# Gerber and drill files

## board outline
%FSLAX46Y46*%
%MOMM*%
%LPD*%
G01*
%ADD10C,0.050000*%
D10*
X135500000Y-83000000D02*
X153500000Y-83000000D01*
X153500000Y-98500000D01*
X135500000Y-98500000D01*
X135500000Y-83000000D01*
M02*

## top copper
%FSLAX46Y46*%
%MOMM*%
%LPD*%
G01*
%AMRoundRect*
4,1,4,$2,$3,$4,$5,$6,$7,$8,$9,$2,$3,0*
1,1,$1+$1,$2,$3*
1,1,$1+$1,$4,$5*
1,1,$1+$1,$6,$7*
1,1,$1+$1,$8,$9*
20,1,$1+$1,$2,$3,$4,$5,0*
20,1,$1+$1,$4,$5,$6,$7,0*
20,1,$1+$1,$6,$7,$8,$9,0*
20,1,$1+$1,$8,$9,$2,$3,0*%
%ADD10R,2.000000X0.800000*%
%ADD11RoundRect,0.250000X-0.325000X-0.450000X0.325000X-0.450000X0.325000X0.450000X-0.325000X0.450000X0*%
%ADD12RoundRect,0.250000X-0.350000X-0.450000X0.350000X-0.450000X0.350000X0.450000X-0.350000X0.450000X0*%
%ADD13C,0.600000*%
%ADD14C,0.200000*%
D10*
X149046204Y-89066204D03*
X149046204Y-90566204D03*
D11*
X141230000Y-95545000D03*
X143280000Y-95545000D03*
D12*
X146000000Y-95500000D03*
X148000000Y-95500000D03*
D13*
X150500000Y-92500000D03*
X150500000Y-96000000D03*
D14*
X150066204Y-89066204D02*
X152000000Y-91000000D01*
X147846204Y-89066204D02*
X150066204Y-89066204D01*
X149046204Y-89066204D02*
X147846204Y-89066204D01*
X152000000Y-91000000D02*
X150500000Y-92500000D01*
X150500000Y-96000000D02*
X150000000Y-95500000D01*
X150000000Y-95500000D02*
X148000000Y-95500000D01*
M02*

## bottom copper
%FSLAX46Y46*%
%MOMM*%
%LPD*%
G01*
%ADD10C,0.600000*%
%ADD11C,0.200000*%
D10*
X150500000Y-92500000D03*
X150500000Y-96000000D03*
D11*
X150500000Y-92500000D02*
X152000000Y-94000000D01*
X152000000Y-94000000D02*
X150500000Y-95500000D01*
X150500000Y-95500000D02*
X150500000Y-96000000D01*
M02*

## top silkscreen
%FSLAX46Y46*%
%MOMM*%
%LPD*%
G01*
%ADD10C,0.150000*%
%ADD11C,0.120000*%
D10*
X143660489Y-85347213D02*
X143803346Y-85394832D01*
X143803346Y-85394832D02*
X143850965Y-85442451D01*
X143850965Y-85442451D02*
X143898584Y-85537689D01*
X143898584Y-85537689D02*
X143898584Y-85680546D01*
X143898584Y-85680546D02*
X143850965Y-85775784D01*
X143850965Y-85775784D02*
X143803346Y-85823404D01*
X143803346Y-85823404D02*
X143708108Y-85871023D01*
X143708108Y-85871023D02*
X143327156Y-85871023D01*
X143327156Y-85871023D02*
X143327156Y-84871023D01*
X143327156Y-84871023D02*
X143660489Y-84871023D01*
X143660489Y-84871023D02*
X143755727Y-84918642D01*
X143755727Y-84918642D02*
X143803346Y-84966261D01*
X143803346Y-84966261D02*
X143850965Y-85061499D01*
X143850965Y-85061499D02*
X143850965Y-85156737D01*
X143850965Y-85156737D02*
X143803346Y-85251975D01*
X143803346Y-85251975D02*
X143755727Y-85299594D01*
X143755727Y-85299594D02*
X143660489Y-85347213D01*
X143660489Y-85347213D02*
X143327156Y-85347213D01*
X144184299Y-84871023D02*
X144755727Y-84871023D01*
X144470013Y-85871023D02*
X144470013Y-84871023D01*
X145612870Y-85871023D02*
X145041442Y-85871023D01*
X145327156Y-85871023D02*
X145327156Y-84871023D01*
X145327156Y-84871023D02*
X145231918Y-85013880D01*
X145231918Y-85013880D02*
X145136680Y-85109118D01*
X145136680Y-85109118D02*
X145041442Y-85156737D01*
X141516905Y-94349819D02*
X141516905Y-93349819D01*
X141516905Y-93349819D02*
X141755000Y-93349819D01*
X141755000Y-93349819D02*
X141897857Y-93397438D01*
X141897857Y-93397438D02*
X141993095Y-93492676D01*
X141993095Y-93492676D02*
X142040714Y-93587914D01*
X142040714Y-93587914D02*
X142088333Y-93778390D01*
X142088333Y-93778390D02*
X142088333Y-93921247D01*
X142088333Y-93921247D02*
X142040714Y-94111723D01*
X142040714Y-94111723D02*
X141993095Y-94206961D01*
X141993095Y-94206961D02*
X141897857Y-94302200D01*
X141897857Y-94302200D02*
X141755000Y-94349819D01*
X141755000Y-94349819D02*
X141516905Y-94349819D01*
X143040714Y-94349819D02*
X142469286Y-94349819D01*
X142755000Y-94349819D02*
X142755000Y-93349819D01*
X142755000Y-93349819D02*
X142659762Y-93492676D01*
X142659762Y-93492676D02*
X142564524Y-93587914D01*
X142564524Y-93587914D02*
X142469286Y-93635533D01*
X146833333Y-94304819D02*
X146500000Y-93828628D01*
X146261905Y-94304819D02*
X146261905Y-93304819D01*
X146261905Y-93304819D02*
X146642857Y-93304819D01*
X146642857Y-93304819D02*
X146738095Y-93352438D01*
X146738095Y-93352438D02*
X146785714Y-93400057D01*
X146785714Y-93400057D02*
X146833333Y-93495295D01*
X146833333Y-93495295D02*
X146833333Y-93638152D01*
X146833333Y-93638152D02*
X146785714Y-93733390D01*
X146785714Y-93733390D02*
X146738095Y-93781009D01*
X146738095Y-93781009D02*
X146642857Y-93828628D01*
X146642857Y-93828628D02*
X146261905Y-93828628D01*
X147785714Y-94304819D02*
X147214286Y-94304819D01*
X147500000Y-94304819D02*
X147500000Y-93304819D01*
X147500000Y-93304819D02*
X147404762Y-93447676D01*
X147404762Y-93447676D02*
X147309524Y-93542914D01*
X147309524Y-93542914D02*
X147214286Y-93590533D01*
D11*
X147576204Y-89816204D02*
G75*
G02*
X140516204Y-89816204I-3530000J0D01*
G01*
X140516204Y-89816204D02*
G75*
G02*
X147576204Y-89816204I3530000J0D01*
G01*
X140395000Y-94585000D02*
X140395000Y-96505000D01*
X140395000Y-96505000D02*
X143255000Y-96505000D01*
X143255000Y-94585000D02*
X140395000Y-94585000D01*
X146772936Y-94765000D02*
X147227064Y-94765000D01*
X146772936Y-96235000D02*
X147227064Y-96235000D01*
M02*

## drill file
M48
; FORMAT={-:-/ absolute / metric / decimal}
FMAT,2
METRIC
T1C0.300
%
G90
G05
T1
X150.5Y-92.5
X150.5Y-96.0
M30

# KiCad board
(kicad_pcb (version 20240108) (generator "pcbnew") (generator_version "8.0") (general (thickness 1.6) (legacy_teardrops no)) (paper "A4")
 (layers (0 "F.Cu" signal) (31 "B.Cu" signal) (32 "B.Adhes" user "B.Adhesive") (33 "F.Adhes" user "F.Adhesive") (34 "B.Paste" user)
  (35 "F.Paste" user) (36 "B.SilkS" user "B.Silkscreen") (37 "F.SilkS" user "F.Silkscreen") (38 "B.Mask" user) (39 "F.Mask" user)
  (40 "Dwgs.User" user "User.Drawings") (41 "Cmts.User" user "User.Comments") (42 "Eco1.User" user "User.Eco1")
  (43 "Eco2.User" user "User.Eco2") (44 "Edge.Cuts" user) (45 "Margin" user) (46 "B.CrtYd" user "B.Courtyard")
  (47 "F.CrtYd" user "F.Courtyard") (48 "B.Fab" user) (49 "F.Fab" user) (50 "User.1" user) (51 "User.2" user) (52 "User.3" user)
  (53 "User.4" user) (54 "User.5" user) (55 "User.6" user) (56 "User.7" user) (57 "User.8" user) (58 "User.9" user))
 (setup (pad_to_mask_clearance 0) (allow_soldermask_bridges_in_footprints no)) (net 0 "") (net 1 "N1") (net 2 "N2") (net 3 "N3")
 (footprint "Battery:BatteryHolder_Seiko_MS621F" (layer "F.Cu") (at 149.046204 89.816204)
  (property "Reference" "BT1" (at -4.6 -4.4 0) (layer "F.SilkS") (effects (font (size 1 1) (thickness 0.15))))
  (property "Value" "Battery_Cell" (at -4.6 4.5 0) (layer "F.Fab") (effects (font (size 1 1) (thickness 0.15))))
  (fp_circle (center -5 0) (end -1.47 0) (stroke (width 0.12) (type solid)) (fill none) (layer "F.SilkS"))
  (pad "1" smd rect (at 0 -0.75) (size 2 0.8) (layers "F.Cu" "F.Paste" "F.Mask") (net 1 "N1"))
  (pad "2" smd rect (at 0 0.75) (size 2 0.8) (layers "F.Cu" "F.Paste" "F.Mask") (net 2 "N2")))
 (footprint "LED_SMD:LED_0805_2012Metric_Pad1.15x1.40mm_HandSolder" (layer "F.Cu") (at 142.255 95.545)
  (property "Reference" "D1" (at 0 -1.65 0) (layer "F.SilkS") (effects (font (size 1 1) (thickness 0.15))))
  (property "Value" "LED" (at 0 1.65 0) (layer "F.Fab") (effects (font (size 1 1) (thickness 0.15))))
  (fp_line (start -1.86 -0.96) (end -1.86 0.96) (stroke (width 0.12) (type solid)) (layer "F.SilkS"))
  (fp_line (start -1.86 0.96) (end 1 0.96) (stroke (width 0.12) (type solid)) (layer "F.SilkS"))
  (fp_line (start 1 -0.96) (end -1.86 -0.96) (stroke (width 0.12) (type solid)) (layer "F.SilkS"))
  (pad "1" smd roundrect (at -1.025 0) (size 1.15 1.4) (layers "F.Cu" "F.Paste" "F.Mask") (roundrect_rratio 0.217391) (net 2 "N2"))
  (pad "2" smd roundrect (at 1.025 0) (size 1.15 1.4) (layers "F.Cu" "F.Paste" "F.Mask") (roundrect_rratio 0.217391) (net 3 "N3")))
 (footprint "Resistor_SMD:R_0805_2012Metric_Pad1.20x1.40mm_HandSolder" (layer "F.Cu") (at 147 95.5)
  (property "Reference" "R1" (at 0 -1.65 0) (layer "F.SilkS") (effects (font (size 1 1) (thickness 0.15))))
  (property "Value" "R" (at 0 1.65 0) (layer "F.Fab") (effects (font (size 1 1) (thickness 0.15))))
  (fp_line (start -0.227064 -0.735) (end 0.227064 -0.735) (stroke (width 0.12) (type solid)) (layer "F.SilkS"))
  (fp_line (start -0.227064 0.735) (end 0.227064 0.735) (stroke (width 0.12) (type solid)) (layer "F.SilkS"))
  (pad "1" smd roundrect (at -1 0) (size 1.2 1.4) (layers "F.Cu" "F.Paste" "F.Mask") (roundrect_rratio 0.208333) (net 3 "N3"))
  (pad "2" smd roundrect (at 1 0) (size 1.2 1.4) (layers "F.Cu" "F.Paste" "F.Mask") (roundrect_rratio 0.208333) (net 1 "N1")))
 (gr_rect (start 135.5 83) (end 153.5 98.5) (stroke (width 0.05) (type default)) (fill none) (layer "Edge.Cuts"))
 (segment (start 150.066204 89.066204) (end 152 91) (width 0.2) (layer "F.Cu") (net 1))
 (segment (start 147.846204 89.066204) (end 150.066204 89.066204) (width 0.2) (layer "F.Cu") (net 1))
 (segment (start 149.046204 89.066204) (end 147.846204 89.066204) (width 0.2) (layer "F.Cu") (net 1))
 (segment (start 152 91) (end 150.5 92.5) (width 0.2) (layer "F.Cu") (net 1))
 (segment (start 150.5 96) (end 150 95.5) (width 0.2) (layer "F.Cu") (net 1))
 (segment (start 150 95.5) (end 148 95.5) (width 0.2) (layer "F.Cu") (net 1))
 (via (at 150.5 92.5) (size 0.6) (drill 0.3) (layers "F.Cu" "B.Cu") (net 1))
 (via (at 150.5 96) (size 0.6) (drill 0.3) (layers "F.Cu" "B.Cu") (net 1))
 (segment (start 150.5 92.5) (end 152 94) (width 0.2) (layer "B.Cu") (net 1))
 (segment (start 152 94) (end 150.5 95.5) (width 0.2) (layer "B.Cu") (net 1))
 (segment (start 150.5 95.5) (end 150.5 96) (width 0.2) (layer "B.Cu") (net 1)))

